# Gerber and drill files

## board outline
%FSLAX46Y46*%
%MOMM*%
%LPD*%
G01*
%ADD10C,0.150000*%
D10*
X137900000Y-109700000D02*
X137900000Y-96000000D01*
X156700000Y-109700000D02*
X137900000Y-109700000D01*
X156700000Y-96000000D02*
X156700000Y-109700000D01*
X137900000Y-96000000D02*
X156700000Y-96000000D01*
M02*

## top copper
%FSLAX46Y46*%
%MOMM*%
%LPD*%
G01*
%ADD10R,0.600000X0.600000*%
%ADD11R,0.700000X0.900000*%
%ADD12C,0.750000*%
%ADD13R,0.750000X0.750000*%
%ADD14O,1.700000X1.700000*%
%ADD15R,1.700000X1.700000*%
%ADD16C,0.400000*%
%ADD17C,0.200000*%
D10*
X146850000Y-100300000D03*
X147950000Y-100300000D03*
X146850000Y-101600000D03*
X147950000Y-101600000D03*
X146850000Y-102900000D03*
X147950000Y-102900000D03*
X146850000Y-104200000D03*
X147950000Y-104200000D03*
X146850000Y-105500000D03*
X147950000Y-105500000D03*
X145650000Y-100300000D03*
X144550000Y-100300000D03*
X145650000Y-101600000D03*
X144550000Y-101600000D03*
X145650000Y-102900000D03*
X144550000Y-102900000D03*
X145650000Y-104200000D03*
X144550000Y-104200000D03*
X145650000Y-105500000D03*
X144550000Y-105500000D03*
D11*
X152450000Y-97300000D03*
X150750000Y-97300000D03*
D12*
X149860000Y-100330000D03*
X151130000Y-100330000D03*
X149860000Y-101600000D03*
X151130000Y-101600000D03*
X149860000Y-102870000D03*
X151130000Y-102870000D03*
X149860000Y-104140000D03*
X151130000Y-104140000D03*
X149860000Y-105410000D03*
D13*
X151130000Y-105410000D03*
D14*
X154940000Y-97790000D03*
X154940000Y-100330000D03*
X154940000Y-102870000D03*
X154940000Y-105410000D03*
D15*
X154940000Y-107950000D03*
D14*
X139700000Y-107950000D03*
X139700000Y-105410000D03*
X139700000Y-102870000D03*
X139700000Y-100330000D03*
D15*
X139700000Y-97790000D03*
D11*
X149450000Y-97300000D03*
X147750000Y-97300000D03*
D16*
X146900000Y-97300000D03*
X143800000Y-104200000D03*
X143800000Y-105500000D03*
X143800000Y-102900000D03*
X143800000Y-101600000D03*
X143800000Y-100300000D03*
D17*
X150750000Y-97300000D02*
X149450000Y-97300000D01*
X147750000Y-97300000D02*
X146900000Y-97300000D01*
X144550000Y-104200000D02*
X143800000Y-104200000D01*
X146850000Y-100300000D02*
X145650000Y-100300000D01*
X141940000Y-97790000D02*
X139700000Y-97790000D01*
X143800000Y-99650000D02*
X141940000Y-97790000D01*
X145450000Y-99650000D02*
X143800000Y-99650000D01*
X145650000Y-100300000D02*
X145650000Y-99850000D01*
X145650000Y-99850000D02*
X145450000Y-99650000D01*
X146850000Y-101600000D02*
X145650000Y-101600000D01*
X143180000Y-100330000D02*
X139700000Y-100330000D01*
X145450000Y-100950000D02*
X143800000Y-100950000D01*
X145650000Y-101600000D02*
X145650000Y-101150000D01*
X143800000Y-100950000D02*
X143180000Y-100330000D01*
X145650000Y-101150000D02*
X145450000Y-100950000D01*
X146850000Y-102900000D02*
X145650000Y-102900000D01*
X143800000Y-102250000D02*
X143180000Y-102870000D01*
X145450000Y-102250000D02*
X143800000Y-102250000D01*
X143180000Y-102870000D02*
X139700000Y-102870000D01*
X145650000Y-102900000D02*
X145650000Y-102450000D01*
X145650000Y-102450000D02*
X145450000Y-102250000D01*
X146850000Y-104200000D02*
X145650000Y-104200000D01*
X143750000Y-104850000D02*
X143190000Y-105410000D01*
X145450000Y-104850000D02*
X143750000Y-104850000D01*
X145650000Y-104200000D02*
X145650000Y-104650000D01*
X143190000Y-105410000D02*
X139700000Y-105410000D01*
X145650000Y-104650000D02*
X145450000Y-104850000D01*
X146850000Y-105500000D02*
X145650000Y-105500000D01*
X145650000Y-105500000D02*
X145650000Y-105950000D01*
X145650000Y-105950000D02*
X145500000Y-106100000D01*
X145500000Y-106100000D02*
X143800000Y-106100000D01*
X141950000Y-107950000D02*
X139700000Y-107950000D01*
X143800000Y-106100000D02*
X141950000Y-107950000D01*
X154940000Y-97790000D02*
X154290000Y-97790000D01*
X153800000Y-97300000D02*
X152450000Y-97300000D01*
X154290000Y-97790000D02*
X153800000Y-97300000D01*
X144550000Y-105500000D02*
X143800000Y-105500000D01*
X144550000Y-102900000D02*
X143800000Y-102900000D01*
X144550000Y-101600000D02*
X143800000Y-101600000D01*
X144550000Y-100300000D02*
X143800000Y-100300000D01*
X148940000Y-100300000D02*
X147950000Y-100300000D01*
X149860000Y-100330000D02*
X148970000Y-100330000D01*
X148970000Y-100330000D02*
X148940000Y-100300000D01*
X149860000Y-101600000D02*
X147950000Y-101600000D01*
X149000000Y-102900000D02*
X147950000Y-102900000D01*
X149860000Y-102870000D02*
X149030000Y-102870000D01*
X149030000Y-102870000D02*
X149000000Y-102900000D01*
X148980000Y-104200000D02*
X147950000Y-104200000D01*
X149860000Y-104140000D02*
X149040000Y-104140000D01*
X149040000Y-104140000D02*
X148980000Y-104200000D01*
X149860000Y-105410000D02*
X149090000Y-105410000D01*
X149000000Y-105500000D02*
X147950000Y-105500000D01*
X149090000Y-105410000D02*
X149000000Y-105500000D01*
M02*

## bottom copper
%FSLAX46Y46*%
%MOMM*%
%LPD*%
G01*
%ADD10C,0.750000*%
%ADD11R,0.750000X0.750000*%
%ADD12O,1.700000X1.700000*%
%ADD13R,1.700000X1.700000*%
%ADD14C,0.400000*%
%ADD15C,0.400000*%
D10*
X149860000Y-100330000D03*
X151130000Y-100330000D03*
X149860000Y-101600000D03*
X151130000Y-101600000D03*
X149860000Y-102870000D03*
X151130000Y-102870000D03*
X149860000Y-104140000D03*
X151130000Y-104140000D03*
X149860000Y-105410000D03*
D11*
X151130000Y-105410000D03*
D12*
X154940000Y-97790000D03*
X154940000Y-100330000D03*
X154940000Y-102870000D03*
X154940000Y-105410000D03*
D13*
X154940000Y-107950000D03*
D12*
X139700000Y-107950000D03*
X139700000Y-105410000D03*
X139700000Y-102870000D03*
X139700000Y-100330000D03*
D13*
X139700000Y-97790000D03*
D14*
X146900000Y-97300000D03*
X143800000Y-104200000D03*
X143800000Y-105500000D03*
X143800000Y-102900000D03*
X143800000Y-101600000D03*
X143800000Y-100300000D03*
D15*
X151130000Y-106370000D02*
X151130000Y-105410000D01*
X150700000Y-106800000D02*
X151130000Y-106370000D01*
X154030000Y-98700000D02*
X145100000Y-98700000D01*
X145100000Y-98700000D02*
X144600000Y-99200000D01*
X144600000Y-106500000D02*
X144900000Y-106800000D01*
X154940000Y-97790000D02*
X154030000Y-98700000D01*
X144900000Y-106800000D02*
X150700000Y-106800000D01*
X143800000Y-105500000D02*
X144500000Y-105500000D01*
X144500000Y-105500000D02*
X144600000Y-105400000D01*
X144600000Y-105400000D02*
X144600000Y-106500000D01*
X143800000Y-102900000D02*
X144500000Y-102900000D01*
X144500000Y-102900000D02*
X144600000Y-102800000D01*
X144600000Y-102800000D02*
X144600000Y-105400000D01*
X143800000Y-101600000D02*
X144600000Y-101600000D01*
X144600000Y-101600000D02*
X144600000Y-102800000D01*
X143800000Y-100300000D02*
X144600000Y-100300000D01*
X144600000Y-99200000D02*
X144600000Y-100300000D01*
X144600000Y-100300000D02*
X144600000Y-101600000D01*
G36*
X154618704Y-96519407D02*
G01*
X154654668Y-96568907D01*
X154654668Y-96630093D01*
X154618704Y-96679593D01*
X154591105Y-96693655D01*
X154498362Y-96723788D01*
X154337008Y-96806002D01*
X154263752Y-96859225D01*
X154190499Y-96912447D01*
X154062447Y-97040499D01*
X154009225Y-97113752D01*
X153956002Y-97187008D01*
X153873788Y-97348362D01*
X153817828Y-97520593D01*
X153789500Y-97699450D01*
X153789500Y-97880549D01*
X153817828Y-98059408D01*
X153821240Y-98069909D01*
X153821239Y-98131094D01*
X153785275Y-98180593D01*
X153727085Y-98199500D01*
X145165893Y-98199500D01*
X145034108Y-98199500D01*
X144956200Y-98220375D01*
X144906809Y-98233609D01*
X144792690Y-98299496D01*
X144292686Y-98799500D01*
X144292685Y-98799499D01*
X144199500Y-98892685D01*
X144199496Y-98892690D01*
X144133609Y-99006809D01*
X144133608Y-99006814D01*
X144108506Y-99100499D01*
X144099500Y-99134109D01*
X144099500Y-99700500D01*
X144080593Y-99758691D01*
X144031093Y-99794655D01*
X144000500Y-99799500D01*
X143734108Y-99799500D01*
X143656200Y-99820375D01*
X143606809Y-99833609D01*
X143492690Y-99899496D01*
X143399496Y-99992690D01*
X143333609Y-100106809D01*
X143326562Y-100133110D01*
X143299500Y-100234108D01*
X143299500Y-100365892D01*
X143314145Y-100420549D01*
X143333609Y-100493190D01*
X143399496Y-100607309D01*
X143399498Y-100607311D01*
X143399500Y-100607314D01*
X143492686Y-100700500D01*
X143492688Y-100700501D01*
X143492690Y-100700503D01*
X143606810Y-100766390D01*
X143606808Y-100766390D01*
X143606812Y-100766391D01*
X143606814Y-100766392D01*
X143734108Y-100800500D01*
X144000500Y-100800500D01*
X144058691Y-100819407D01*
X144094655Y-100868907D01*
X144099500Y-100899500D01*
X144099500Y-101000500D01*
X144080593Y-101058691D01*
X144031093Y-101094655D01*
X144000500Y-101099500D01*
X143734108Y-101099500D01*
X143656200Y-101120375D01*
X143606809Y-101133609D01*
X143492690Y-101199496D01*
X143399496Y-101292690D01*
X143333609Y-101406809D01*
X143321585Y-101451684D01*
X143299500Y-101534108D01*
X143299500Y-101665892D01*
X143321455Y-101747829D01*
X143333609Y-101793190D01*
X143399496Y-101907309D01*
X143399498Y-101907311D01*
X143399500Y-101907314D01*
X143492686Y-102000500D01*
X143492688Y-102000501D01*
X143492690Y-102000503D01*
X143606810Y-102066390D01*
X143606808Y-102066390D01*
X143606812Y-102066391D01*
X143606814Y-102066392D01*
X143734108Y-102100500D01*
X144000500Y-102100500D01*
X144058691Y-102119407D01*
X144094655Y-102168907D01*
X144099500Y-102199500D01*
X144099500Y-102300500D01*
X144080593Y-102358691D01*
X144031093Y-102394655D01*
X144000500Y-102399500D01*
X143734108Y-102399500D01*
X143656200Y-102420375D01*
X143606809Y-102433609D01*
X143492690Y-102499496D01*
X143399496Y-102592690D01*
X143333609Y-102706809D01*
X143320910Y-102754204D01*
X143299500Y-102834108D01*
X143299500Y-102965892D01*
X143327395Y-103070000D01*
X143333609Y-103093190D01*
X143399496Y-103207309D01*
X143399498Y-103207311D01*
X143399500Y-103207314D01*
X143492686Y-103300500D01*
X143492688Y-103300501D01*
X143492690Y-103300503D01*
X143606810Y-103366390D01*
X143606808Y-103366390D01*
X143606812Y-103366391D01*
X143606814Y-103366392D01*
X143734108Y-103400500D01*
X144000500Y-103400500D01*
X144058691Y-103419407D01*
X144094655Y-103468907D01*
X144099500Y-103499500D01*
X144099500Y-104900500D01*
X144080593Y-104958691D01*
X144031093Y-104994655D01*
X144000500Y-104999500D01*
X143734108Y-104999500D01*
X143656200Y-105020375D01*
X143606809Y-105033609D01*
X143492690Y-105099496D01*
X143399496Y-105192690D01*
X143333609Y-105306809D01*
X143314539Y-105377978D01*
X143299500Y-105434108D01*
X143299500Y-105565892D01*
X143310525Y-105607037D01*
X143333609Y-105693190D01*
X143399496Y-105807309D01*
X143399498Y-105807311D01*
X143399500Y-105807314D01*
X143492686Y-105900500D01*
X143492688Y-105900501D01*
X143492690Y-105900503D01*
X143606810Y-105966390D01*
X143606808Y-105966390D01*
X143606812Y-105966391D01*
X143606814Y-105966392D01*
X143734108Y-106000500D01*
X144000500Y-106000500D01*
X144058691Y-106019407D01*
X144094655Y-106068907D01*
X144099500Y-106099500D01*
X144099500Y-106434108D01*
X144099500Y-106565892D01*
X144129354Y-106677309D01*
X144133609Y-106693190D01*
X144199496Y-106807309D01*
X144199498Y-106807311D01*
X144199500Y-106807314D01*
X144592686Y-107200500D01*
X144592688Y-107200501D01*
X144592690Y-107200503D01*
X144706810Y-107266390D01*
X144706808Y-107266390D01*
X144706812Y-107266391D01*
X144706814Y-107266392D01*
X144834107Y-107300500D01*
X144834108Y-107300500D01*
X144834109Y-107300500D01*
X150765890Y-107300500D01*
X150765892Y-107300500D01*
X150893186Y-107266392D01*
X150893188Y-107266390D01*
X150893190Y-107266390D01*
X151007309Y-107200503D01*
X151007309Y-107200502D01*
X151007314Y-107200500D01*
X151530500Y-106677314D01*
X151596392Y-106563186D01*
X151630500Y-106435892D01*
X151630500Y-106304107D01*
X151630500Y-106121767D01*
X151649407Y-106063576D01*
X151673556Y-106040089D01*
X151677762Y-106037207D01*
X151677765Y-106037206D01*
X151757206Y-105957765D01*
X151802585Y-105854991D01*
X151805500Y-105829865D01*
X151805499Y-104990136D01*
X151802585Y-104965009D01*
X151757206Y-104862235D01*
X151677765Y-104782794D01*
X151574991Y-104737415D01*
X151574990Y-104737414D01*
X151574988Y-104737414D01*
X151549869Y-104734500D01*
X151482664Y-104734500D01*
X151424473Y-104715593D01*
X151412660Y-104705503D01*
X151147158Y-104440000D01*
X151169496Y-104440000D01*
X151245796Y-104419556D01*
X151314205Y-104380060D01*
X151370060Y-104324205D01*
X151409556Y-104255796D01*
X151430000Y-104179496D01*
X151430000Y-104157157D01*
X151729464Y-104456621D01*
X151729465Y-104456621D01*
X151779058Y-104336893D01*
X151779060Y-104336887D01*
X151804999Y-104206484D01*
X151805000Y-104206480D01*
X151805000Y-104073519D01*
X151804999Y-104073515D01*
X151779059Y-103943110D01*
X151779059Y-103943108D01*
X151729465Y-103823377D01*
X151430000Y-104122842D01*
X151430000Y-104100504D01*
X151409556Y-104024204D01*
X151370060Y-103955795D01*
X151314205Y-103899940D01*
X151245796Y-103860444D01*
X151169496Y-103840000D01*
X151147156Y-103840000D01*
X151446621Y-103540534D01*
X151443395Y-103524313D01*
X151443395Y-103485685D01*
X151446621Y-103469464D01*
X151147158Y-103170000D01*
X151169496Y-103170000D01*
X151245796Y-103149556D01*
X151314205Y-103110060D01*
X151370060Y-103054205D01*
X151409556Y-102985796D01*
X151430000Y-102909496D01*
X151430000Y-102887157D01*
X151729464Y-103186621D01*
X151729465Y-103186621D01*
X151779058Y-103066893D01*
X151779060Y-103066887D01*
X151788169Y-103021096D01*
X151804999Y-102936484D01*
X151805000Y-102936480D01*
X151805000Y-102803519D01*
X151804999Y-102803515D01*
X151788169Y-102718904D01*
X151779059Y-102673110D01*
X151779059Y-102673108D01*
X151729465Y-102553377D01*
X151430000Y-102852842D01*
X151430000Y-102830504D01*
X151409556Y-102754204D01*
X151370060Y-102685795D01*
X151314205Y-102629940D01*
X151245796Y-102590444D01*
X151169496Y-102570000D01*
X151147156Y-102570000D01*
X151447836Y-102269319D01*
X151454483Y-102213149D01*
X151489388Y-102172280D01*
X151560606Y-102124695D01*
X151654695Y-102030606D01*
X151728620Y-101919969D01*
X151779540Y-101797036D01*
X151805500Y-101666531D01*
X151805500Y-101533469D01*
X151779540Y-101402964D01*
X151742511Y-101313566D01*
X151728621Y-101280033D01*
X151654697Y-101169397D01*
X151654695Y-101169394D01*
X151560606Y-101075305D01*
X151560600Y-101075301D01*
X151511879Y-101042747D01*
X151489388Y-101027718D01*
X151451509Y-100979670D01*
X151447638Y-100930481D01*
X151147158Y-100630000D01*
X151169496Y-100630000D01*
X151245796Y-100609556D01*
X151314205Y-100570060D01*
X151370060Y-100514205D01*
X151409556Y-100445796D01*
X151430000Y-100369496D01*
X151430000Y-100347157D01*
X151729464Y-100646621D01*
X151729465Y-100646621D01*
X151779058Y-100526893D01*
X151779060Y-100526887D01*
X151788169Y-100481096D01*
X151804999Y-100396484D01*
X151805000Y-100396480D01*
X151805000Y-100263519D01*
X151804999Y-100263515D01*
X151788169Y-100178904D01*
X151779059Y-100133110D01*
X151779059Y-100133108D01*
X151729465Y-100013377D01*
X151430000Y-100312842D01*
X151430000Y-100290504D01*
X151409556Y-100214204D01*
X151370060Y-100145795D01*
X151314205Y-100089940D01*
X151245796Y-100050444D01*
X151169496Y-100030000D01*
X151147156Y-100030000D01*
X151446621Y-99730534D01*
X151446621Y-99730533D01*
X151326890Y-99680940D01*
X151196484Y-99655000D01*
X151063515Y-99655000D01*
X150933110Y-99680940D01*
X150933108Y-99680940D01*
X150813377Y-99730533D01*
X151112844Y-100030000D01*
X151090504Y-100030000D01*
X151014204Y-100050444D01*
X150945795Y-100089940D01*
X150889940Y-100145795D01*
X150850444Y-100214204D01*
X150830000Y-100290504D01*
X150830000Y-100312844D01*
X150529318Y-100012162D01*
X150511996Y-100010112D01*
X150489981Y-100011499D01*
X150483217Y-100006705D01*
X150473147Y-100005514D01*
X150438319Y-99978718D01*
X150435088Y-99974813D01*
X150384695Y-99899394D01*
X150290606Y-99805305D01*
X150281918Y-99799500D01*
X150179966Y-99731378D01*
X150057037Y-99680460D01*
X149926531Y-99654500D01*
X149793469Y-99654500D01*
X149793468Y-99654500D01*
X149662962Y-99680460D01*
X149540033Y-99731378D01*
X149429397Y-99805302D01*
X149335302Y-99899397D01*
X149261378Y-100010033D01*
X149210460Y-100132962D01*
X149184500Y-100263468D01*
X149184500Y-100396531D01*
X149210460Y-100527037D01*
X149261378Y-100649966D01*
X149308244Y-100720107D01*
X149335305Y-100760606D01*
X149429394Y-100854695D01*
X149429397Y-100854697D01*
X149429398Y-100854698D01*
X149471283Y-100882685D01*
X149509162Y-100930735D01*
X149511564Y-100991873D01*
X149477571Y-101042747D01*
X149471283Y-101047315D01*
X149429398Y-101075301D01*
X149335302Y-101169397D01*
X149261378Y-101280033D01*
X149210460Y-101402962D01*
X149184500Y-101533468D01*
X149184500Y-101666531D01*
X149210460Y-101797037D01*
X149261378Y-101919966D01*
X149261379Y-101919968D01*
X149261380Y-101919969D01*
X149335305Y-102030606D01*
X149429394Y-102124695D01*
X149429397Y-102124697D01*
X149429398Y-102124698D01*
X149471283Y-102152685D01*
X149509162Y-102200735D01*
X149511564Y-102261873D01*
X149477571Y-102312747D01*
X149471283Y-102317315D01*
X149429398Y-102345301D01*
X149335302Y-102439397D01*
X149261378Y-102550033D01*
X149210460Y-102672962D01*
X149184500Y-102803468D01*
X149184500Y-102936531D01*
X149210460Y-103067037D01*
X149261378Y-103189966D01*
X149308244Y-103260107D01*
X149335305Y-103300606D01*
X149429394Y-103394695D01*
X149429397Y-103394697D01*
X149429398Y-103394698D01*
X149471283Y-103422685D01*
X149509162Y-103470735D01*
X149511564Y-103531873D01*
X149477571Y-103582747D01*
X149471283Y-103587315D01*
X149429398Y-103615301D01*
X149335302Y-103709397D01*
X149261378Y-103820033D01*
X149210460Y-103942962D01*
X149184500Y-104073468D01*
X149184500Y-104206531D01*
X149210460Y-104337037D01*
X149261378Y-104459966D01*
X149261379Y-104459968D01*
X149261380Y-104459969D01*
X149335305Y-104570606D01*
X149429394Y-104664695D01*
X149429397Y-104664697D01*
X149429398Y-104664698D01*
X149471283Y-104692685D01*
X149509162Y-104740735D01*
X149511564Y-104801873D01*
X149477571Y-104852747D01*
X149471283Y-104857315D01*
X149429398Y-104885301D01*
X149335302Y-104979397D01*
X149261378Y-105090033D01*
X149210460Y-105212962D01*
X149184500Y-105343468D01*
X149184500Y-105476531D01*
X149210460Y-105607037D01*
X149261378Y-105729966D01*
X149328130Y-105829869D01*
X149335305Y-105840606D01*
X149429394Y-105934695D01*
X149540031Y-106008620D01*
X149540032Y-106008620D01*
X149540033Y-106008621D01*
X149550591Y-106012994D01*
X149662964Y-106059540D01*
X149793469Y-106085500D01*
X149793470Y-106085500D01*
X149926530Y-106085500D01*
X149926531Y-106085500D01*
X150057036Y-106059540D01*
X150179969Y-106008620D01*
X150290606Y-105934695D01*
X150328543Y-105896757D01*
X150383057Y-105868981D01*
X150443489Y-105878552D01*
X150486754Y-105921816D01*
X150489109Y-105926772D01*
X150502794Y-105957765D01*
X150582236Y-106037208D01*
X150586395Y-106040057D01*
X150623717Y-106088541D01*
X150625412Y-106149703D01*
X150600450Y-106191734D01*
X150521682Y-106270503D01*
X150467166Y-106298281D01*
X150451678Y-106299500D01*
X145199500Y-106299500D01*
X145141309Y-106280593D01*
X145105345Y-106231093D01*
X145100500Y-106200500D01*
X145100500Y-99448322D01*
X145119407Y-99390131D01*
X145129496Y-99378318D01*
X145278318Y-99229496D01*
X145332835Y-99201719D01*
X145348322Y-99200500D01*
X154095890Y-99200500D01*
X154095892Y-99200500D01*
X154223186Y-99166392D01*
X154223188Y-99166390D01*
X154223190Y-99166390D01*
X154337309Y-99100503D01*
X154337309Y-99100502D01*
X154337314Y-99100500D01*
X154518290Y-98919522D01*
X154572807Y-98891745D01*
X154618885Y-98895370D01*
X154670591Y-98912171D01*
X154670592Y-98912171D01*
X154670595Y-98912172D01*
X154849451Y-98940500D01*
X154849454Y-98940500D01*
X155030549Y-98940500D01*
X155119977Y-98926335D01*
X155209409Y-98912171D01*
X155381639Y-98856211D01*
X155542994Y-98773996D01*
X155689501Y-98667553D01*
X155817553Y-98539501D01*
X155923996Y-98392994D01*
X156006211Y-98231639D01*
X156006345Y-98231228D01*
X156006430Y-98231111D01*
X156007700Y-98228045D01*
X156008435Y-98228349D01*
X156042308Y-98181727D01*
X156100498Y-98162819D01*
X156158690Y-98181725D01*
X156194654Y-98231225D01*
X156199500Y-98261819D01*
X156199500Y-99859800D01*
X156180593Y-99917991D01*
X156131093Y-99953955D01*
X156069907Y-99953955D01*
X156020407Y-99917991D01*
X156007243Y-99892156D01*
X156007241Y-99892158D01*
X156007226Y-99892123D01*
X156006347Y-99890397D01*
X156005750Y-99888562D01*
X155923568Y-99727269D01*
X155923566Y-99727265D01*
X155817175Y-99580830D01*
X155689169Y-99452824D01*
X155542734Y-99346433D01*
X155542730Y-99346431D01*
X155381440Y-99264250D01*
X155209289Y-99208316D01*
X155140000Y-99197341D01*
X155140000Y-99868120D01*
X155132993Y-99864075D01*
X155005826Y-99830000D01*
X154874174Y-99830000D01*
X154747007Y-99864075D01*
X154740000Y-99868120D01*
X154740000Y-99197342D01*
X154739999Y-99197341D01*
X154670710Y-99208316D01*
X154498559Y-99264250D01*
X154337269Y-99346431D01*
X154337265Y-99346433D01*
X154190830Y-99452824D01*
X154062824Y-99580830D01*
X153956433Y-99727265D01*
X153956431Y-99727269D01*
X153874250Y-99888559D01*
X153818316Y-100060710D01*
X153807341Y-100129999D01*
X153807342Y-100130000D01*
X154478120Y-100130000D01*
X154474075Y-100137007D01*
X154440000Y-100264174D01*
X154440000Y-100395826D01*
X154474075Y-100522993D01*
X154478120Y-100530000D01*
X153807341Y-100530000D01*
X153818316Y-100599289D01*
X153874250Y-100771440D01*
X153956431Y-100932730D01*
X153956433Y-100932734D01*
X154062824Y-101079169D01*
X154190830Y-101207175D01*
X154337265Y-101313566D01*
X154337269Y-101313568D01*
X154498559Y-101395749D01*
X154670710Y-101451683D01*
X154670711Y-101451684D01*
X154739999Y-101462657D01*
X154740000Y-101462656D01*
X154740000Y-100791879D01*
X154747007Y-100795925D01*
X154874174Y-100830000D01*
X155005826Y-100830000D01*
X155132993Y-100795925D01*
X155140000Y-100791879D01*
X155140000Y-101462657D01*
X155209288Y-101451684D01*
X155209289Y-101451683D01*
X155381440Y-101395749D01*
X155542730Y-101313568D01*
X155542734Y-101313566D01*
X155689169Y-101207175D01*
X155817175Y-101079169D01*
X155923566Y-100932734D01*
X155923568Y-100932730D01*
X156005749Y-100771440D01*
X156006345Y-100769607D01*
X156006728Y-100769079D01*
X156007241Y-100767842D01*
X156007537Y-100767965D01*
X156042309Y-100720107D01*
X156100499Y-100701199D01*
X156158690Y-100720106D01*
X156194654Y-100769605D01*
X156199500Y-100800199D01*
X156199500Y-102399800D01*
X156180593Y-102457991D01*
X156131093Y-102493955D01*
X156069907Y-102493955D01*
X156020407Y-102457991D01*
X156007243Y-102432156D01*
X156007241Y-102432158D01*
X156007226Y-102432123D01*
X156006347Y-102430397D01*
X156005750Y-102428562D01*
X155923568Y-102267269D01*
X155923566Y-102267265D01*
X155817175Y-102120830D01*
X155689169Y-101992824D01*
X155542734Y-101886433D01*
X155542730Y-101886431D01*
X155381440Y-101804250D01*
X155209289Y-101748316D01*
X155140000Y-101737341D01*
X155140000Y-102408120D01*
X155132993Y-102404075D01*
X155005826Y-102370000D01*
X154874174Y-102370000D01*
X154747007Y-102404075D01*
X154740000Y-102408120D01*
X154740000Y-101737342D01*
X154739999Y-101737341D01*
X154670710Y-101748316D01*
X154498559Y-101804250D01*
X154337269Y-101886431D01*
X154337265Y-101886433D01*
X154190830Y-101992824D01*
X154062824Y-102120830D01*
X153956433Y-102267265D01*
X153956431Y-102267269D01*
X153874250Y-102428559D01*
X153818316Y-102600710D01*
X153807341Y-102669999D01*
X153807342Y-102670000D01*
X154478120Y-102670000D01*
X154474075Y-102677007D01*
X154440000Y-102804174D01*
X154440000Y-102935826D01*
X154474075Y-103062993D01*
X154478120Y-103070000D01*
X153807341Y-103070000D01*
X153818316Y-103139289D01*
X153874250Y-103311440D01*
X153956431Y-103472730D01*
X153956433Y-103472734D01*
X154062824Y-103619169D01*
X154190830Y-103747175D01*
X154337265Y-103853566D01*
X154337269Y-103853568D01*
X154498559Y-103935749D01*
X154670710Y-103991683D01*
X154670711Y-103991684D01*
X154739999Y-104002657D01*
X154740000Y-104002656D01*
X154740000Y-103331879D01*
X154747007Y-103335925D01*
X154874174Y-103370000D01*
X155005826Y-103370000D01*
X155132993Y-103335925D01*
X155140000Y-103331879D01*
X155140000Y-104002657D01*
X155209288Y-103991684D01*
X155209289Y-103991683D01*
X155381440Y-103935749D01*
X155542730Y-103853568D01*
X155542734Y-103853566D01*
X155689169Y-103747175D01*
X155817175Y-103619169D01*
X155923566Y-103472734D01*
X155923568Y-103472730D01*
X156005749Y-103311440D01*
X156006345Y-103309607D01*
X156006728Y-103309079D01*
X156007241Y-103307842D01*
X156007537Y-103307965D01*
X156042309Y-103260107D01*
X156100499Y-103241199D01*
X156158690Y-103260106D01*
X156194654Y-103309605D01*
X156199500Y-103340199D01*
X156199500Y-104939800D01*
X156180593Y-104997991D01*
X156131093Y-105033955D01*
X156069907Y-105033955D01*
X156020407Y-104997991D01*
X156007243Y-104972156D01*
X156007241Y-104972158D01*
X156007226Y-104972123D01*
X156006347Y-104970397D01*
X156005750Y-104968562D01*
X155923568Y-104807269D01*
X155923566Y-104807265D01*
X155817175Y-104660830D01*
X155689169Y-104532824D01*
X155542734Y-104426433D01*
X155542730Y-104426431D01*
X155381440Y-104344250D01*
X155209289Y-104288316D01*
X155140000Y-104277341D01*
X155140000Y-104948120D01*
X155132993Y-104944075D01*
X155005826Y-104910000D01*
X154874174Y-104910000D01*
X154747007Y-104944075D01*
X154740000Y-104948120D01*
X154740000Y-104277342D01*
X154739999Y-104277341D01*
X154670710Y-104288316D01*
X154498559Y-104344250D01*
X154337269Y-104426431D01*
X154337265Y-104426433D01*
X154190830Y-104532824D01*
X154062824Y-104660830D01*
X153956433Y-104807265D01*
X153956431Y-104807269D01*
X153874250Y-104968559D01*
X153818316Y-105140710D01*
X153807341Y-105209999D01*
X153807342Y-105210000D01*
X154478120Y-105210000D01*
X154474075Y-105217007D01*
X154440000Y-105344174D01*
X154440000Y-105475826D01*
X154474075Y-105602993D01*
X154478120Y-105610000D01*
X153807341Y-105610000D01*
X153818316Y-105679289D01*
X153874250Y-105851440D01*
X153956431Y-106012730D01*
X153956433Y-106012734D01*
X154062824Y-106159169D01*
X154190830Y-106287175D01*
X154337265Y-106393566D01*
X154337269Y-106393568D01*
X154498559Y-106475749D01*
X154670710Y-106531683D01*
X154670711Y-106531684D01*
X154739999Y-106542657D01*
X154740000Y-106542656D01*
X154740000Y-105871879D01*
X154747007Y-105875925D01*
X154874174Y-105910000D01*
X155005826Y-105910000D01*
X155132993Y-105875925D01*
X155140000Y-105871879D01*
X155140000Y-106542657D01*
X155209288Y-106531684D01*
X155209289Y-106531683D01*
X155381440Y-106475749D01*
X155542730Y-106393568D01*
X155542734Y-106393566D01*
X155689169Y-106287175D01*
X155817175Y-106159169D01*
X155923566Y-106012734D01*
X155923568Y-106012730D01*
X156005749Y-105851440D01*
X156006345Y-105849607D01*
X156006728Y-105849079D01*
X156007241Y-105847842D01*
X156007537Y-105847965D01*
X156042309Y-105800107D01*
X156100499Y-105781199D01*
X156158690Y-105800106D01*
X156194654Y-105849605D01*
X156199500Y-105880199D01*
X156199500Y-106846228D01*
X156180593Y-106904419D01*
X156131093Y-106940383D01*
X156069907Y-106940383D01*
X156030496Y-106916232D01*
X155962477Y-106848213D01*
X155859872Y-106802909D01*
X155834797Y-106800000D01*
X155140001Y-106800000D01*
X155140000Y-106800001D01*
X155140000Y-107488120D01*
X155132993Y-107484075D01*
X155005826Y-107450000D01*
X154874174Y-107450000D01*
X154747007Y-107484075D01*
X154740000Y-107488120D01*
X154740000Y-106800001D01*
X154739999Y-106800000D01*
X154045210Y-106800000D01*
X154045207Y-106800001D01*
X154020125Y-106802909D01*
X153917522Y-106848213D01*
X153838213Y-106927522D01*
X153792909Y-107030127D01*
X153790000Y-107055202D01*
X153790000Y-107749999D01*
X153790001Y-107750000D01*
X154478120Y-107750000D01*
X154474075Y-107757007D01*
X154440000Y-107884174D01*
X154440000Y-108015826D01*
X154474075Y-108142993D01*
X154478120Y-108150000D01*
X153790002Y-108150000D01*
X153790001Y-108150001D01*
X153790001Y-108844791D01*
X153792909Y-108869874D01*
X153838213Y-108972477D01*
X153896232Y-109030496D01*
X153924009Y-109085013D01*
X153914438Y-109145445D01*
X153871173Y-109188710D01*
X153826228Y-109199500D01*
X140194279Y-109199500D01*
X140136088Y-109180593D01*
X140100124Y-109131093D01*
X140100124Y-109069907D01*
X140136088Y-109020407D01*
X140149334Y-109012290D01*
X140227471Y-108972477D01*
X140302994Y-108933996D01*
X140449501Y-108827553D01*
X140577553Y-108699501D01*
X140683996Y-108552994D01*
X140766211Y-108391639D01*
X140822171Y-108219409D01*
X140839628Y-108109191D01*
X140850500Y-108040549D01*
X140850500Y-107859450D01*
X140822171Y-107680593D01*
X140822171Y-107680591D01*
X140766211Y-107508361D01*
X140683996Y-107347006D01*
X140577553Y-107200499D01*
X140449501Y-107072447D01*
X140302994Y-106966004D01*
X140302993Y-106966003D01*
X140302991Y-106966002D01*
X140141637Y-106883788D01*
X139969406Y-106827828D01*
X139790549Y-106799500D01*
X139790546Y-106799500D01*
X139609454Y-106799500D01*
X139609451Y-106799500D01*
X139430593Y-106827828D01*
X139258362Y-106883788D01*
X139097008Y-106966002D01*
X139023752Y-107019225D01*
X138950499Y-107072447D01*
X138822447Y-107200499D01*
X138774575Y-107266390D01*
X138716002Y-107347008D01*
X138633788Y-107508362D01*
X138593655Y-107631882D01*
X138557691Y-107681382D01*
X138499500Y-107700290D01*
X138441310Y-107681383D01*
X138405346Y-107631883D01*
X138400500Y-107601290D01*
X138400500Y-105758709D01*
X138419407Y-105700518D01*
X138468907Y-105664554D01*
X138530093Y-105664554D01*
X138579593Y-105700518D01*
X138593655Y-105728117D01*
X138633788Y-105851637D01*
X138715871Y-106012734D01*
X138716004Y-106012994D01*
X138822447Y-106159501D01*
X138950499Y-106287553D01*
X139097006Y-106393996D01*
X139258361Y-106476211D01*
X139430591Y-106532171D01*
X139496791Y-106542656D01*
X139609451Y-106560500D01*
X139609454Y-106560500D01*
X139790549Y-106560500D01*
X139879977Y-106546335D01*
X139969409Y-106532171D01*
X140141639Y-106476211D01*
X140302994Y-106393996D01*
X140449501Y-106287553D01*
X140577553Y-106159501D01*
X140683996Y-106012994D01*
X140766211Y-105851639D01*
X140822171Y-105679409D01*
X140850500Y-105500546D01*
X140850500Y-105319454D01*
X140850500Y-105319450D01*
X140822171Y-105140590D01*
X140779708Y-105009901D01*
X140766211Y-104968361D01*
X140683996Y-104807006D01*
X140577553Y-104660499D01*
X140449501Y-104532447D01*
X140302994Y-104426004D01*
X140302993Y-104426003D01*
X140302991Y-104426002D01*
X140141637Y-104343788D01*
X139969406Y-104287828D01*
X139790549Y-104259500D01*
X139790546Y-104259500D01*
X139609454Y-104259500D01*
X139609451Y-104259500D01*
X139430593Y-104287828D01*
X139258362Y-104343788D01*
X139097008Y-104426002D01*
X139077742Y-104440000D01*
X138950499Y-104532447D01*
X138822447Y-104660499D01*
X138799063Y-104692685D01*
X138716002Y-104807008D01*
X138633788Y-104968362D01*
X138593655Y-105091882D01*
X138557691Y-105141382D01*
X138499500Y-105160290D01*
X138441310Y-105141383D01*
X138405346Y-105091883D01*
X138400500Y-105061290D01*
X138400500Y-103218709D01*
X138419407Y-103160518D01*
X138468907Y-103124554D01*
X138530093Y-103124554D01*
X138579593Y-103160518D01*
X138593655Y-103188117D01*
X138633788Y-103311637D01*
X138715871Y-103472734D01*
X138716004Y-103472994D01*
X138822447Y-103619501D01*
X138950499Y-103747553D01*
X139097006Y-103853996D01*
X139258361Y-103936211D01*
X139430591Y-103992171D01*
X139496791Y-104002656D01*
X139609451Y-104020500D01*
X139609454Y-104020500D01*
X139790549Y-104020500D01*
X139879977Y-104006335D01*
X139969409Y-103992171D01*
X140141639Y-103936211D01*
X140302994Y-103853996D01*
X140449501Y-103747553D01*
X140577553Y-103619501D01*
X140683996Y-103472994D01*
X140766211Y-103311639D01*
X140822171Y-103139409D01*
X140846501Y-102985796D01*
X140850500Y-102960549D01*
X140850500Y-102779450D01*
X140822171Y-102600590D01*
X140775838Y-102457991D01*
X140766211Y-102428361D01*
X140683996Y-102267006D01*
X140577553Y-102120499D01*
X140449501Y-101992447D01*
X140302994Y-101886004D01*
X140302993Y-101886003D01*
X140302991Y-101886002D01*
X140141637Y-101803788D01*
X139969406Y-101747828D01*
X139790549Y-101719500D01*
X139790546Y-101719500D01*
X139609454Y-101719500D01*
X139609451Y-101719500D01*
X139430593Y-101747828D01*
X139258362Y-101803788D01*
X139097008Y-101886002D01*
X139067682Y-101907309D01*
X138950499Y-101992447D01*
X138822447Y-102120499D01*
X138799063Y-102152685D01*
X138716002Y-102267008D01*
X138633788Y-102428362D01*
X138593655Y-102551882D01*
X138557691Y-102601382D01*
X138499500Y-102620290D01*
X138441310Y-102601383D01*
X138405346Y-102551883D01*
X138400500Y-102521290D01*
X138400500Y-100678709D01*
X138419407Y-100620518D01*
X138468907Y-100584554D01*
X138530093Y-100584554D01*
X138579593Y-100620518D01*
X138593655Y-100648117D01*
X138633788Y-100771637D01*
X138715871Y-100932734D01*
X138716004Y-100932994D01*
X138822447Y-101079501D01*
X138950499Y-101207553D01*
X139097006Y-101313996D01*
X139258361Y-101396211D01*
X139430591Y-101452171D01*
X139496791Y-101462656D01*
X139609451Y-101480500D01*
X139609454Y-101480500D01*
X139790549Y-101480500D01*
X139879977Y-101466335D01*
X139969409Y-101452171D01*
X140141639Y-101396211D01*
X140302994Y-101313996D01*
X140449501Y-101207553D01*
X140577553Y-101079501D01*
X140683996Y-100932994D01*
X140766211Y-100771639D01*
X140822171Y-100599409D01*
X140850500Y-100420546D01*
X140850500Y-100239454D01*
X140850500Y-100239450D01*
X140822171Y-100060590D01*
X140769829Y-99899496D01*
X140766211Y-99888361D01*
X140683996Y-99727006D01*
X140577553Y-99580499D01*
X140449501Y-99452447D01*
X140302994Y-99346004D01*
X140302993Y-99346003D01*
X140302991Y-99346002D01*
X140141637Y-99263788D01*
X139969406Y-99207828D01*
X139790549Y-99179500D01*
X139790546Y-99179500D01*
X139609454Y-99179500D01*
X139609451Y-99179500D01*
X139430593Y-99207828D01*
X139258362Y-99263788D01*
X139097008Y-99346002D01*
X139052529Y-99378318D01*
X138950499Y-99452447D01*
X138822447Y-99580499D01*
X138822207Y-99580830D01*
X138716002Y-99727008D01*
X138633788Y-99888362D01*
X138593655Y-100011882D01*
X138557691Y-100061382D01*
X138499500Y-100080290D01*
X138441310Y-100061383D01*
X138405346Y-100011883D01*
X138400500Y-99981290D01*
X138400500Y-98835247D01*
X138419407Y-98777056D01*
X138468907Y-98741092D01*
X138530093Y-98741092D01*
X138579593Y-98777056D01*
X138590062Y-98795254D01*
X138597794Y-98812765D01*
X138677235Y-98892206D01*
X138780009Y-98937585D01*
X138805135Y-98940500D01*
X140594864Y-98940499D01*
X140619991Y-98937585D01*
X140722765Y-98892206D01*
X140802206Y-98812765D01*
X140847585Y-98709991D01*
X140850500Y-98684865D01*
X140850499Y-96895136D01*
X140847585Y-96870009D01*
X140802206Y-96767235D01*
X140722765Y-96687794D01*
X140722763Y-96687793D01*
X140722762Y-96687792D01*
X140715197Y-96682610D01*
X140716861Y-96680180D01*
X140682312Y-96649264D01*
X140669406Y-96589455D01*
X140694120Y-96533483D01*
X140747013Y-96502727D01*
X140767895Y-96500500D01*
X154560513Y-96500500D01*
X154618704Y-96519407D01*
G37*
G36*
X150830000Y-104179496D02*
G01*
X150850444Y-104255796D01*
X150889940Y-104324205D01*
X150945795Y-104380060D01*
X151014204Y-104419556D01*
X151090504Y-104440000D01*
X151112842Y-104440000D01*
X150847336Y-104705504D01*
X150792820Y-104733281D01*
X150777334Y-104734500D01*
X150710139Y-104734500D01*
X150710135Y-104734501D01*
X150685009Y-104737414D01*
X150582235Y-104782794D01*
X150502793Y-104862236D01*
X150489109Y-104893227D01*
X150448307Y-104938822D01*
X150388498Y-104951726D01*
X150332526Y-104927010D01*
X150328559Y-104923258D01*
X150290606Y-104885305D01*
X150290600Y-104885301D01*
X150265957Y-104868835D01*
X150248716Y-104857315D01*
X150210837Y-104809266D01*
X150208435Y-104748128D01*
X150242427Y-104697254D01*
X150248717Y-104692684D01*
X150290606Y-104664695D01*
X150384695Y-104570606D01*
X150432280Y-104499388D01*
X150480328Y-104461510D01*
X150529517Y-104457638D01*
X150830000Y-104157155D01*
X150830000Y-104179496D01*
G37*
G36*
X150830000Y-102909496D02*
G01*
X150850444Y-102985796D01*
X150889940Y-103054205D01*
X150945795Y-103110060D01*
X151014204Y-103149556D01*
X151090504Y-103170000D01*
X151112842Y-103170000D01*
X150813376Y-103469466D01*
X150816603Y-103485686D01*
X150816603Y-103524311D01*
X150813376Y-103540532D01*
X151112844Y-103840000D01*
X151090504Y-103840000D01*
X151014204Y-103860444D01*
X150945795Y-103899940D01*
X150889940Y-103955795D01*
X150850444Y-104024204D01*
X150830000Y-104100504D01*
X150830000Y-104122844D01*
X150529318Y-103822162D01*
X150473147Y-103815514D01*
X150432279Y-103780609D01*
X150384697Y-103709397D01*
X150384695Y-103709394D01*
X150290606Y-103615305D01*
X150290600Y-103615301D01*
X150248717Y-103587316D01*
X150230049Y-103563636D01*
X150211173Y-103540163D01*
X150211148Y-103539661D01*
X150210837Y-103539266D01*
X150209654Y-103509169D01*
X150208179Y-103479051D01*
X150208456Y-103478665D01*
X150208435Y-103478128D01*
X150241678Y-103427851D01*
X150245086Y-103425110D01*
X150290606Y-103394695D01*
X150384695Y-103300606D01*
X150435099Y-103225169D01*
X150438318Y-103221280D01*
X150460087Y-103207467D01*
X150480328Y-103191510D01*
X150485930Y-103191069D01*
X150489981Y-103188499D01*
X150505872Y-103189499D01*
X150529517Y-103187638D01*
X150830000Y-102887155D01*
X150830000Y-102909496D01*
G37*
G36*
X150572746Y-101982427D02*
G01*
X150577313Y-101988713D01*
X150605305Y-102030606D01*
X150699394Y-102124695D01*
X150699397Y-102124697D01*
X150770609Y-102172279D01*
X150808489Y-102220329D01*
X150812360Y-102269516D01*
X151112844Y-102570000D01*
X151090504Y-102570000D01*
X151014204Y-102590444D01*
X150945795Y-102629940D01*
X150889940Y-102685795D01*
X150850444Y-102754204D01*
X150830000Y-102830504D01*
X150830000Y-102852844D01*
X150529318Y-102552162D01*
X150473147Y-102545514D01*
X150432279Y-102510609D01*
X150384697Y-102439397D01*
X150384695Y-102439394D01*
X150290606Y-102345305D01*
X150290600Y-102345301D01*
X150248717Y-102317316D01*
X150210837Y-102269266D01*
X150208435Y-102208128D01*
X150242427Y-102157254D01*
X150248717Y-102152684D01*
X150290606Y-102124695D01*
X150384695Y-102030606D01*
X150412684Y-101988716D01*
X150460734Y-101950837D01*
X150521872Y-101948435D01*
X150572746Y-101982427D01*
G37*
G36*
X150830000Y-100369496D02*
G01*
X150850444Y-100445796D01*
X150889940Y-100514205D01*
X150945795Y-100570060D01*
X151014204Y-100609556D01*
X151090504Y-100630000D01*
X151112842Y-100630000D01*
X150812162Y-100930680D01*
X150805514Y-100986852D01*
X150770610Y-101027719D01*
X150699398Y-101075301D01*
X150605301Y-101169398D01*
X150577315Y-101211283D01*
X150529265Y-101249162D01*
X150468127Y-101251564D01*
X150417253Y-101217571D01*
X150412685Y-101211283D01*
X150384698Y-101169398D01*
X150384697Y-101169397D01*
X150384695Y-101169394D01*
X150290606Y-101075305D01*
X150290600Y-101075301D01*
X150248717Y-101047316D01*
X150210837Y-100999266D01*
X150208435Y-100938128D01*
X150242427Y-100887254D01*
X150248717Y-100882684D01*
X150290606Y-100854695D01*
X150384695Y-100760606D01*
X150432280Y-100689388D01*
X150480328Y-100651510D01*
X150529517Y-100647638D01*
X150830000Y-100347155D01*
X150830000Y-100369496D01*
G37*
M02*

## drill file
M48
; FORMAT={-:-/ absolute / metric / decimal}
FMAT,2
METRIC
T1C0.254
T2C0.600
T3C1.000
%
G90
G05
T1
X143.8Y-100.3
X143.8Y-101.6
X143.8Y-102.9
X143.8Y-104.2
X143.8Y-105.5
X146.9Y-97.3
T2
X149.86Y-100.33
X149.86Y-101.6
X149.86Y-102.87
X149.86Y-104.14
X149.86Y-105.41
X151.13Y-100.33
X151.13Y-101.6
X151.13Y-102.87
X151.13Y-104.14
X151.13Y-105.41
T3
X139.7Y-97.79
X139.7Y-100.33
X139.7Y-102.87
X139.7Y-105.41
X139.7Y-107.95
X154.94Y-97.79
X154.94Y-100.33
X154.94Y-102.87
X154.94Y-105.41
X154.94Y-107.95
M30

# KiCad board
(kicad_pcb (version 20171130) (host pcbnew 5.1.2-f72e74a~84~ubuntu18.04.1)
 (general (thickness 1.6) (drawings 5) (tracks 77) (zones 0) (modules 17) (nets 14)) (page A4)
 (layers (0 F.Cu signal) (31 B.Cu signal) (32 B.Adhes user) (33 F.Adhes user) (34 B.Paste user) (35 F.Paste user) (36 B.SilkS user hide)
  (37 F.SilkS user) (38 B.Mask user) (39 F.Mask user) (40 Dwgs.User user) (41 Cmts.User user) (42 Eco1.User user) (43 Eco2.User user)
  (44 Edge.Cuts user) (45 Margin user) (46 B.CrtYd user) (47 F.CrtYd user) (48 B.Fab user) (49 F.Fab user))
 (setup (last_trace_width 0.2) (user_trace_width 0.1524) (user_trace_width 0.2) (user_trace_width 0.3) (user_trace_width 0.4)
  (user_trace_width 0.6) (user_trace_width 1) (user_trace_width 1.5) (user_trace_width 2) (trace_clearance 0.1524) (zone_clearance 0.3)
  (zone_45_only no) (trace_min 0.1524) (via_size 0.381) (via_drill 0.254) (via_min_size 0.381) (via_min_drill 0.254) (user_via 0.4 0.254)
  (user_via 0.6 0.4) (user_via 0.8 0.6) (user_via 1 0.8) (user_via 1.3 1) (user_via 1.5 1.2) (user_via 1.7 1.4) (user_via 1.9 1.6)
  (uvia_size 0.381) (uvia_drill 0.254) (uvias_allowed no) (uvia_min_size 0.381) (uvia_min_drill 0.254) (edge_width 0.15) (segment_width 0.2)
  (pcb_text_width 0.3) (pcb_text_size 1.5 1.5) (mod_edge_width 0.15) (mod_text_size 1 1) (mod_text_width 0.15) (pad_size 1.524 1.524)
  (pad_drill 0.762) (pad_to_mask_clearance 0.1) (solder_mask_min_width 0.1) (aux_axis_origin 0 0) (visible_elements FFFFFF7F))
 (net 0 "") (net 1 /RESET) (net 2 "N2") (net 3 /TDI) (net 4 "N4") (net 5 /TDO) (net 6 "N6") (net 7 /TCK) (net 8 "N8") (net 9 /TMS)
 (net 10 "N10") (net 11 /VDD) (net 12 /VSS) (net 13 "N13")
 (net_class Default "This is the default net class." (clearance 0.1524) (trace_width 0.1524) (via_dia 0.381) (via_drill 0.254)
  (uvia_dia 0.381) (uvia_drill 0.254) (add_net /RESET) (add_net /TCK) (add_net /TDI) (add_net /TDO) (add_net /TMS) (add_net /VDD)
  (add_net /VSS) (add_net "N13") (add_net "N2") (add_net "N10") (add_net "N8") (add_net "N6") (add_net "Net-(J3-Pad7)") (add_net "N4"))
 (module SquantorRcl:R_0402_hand (layer F.Cu) (at 147.4 100.3 180)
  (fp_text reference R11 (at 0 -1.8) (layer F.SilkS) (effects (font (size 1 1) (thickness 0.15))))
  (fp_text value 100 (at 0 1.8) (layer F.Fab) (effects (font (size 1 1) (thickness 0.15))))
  (pad 2 smd rect (at 0.55 0 180) (size 0.6 0.6) (layers F.Cu F.Paste F.Mask) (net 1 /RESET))
  (pad 1 smd rect (at -0.55 0 180) (size 0.6 0.6) (layers F.Cu F.Paste F.Mask) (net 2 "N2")))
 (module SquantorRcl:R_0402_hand (layer F.Cu) (at 147.4 101.6 180)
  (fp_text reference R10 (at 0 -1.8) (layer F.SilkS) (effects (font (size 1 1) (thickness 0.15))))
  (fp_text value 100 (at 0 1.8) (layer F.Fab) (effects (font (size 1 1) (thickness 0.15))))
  (pad 2 smd rect (at 0.55 0 180) (size 0.6 0.6) (layers F.Cu F.Paste F.Mask) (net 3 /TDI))
  (pad 1 smd rect (at -0.55 0 180) (size 0.6 0.6) (layers F.Cu F.Paste F.Mask) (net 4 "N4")))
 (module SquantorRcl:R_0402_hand (layer F.Cu) (at 147.4 102.9 180)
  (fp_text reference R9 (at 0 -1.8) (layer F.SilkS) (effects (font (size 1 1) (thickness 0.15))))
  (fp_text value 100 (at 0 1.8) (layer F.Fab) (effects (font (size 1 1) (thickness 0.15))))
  (pad 2 smd rect (at 0.55 0 180) (size 0.6 0.6) (layers F.Cu F.Paste F.Mask) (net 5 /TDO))
  (pad 1 smd rect (at -0.55 0 180) (size 0.6 0.6) (layers F.Cu F.Paste F.Mask) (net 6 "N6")))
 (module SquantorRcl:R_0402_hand (layer F.Cu) (at 147.4 104.2 180)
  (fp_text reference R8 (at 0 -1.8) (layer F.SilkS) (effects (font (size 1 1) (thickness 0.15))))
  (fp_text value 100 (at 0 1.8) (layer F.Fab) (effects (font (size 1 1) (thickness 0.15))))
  (pad 2 smd rect (at 0.55 0 180) (size 0.6 0.6) (layers F.Cu F.Paste F.Mask) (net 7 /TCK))
  (pad 1 smd rect (at -0.55 0 180) (size 0.6 0.6) (layers F.Cu F.Paste F.Mask) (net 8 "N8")))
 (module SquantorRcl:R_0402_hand (layer F.Cu) (at 147.4 105.5 180)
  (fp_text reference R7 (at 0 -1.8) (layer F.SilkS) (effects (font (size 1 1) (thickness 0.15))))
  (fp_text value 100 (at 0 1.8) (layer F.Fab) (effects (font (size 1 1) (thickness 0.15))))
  (pad 2 smd rect (at 0.55 0 180) (size 0.6 0.6) (layers F.Cu F.Paste F.Mask) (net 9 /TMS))
  (pad 1 smd rect (at -0.55 0 180) (size 0.6 0.6) (layers F.Cu F.Paste F.Mask) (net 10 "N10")))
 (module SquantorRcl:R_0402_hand (layer F.Cu) (at 145.1 100.3)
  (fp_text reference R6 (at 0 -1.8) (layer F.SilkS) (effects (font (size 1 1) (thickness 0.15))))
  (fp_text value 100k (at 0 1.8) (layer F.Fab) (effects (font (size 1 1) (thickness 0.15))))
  (pad 2 smd rect (at 0.55 0) (size 0.6 0.6) (layers F.Cu F.Paste F.Mask) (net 1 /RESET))
  (pad 1 smd rect (at -0.55 0) (size 0.6 0.6) (layers F.Cu F.Paste F.Mask) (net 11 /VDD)))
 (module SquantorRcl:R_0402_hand (layer F.Cu) (at 145.1 101.6)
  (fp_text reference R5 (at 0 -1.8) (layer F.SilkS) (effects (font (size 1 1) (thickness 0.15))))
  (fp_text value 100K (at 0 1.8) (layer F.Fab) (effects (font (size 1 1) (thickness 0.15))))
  (pad 2 smd rect (at 0.55 0) (size 0.6 0.6) (layers F.Cu F.Paste F.Mask) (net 3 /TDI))
  (pad 1 smd rect (at -0.55 0) (size 0.6 0.6) (layers F.Cu F.Paste F.Mask) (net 11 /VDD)))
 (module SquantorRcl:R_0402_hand (layer F.Cu) (at 145.1 102.9)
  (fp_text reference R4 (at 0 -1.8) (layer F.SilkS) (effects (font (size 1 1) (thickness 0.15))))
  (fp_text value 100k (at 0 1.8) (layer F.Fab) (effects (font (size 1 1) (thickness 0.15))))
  (pad 2 smd rect (at 0.55 0) (size 0.6 0.6) (layers F.Cu F.Paste F.Mask) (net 5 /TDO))
  (pad 1 smd rect (at -0.55 0) (size 0.6 0.6) (layers F.Cu F.Paste F.Mask) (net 11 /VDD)))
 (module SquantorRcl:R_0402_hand (layer F.Cu) (at 145.1 104.2)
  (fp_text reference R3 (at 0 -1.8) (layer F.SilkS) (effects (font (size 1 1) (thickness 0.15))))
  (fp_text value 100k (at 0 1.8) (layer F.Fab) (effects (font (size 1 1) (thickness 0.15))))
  (pad 2 smd rect (at 0.55 0) (size 0.6 0.6) (layers F.Cu F.Paste F.Mask) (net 7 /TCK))
  (pad 1 smd rect (at -0.55 0) (size 0.6 0.6) (layers F.Cu F.Paste F.Mask) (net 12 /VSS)))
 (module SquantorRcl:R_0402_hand (layer F.Cu) (at 145.1 105.5)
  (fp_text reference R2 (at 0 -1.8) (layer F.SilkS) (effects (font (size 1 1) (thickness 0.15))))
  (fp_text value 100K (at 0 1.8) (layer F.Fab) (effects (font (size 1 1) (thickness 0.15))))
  (pad 2 smd rect (at 0.55 0) (size 0.6 0.6) (layers F.Cu F.Paste F.Mask) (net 9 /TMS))
  (pad 1 smd rect (at -0.55 0) (size 0.6 0.6) (layers F.Cu F.Paste F.Mask) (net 11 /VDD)))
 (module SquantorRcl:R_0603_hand (layer F.Cu) (at 151.6 97.3)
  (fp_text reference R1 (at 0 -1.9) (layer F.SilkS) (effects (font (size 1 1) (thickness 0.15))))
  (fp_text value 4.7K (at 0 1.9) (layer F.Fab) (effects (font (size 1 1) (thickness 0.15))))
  (pad 2 smd rect (at 0.85 0) (size 0.7 0.9) (layers F.Cu F.Paste F.Mask) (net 11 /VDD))
  (pad 1 smd rect (at -0.85 0) (size 0.7 0.9) (layers F.Cu F.Paste F.Mask) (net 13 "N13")))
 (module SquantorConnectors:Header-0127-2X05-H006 (layer F.Cu) (at 150.495 102.87 90)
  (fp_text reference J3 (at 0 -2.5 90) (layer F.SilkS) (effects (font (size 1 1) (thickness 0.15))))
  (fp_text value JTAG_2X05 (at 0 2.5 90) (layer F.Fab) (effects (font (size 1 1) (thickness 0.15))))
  (pad 10 thru_hole circle (at 2.54 -0.635 90) (size 0.75 0.75) (drill 0.6) (layers *.Cu *.Mask) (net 2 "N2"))
  (pad 9 thru_hole circle (at 2.54 0.635 90) (size 0.75 0.75) (drill 0.6) (layers *.Cu *.Mask) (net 12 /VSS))
  (pad 8 thru_hole circle (at 1.27 -0.635 90) (size 0.75 0.75) (drill 0.6) (layers *.Cu *.Mask) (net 4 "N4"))
  (pad 7 thru_hole circle (at 1.27 0.635 90) (size 0.75 0.75) (drill 0.6) (layers *.Cu *.Mask))
  (pad 6 thru_hole circle (at 0 -0.635 90) (size 0.75 0.75) (drill 0.6) (layers *.Cu *.Mask) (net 6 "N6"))
  (pad 5 thru_hole circle (at 0 0.635 90) (size 0.75 0.75) (drill 0.6) (layers *.Cu *.Mask) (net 12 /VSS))
  (pad 4 thru_hole circle (at -1.27 -0.635 90) (size 0.75 0.75) (drill 0.6) (layers *.Cu *.Mask) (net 8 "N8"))
  (pad 3 thru_hole circle (at -1.27 0.635 90) (size 0.75 0.75) (drill 0.6) (layers *.Cu *.Mask) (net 12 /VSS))
  (pad 2 thru_hole circle (at -2.54 -0.635 90) (size 0.75 0.75) (drill 0.6) (layers *.Cu *.Mask) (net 10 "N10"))
  (pad 1 thru_hole rect (at -2.54 0.635 90) (size 0.75 0.75) (drill 0.6) (layers *.Cu *.Mask) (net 11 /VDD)))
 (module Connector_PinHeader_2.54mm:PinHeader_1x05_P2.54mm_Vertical (layer F.Cu) (at 154.94 107.95 180)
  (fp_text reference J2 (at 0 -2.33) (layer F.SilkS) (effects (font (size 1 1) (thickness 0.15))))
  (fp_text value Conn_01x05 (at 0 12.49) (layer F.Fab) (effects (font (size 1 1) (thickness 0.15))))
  (pad 5 thru_hole oval (at 0 10.16 180) (size 1.7 1.7) (drill 1) (layers *.Cu *.Mask) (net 11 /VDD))
  (pad 4 thru_hole oval (at 0 7.62 180) (size 1.7 1.7) (drill 1) (layers *.Cu *.Mask) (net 12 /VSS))
  (pad 3 thru_hole oval (at 0 5.08 180) (size 1.7 1.7) (drill 1) (layers *.Cu *.Mask) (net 12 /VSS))
  (pad 2 thru_hole oval (at 0 2.54 180) (size 1.7 1.7) (drill 1) (layers *.Cu *.Mask) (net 12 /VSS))
  (pad 1 thru_hole rect (at 0 0 180) (size 1.7 1.7) (drill 1) (layers *.Cu *.Mask) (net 12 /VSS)))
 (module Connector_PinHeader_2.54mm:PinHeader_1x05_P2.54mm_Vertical (layer F.Cu) (at 139.7 97.79)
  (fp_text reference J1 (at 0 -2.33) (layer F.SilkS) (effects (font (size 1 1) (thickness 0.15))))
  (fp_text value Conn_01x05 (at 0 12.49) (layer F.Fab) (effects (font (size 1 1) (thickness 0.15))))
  (pad 5 thru_hole oval (at 0 10.16) (size 1.7 1.7) (drill 1) (layers *.Cu *.Mask) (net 9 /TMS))
  (pad 4 thru_hole oval (at 0 7.62) (size 1.7 1.7) (drill 1) (layers *.Cu *.Mask) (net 7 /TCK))
  (pad 3 thru_hole oval (at 0 5.08) (size 1.7 1.7) (drill 1) (layers *.Cu *.Mask) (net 5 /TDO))
  (pad 2 thru_hole oval (at 0 2.54) (size 1.7 1.7) (drill 1) (layers *.Cu *.Mask) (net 3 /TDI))
  (pad 1 thru_hole rect (at 0 0) (size 1.7 1.7) (drill 1) (layers *.Cu *.Mask) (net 1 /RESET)))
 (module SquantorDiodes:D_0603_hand (layer F.Cu) (at 148.6 97.3)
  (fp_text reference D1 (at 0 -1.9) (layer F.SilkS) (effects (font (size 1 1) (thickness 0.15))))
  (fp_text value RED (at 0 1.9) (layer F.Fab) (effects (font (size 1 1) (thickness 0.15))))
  (pad 2 smd rect (at 0.85 0) (size 0.7 0.9) (layers F.Cu F.Paste F.Mask) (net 13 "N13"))
  (pad 1 smd rect (at -0.85 0) (size 0.7 0.9) (layers F.Cu F.Paste F.Mask) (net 12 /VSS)))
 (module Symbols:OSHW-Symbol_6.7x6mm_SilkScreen (layer B.Cu) (at 148 101)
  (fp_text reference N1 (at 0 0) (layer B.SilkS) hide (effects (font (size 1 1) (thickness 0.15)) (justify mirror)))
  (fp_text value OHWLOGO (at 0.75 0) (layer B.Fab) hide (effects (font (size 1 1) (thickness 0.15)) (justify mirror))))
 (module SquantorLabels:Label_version (layer B.Cu) (at 148.9 104.8)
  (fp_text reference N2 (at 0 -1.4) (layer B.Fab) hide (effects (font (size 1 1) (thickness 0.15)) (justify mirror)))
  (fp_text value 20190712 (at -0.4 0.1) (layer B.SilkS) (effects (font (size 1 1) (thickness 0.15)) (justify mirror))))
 (gr_line (start 137.9 109.7) (end 137.9 96) (layer Edge.Cuts) (width 0.15))
 (gr_line (start 156.7 109.7) (end 137.9 109.7) (layer Edge.Cuts) (width 0.15))
 (gr_line (start 156.7 96) (end 156.7 109.7) (layer Edge.Cuts) (width 0.15))
 (gr_line (start 137.9 96) (end 156.7 96) (layer Edge.Cuts) (width 0.15))
 (segment (start 150.75 97.3) (end 149.45 97.3) (width 0.2) (layer F.Cu) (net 13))
 (via (at 146.9 97.3) (size 0.4) (drill 0.254) (layers F.Cu B.Cu) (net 12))
 (segment (start 147.75 97.3) (end 146.9 97.3) (width 0.2) (layer F.Cu) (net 12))
 (via (at 143.8 104.2) (size 0.4) (drill 0.254) (layers F.Cu B.Cu) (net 12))
 (segment (start 144.55 104.2) (end 143.8 104.2) (width 0.2) (layer F.Cu) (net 12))
 (segment (start 146.85 100.3) (end 145.65 100.3) (width 0.2) (layer F.Cu) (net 1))
 (segment (start 141.94 97.79) (end 139.7 97.79) (width 0.2) (layer F.Cu) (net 1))
 (segment (start 143.8 99.65) (end 141.94 97.79) (width 0.2) (layer F.Cu) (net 1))
 (segment (start 145.45 99.65) (end 143.8 99.65) (width 0.2) (layer F.Cu) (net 1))
 (segment (start 145.65 100.3) (end 145.65 99.85) (width 0.2) (layer F.Cu) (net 1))
 (segment (start 145.65 99.85) (end 145.45 99.65) (width 0.2) (layer F.Cu) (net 1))
 (segment (start 146.85 101.6) (end 145.65 101.6) (width 0.2) (layer F.Cu) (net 3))
 (segment (start 143.18 100.33) (end 139.7 100.33) (width 0.2) (layer F.Cu) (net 3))
 (segment (start 145.45 100.95) (end 143.8 100.95) (width 0.2) (layer F.Cu) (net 3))
 (segment (start 145.65 101.6) (end 145.65 101.15) (width 0.2) (layer F.Cu) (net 3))
 (segment (start 143.8 100.95) (end 143.18 100.33) (width 0.2) (layer F.Cu) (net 3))
 (segment (start 145.65 101.15) (end 145.45 100.95) (width 0.2) (layer F.Cu) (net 3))
 (segment (start 146.85 102.9) (end 145.65 102.9) (width 0.2) (layer F.Cu) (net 5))
 (segment (start 143.8 102.25) (end 143.18 102.87) (width 0.2) (layer F.Cu) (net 5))
 (segment (start 145.45 102.25) (end 143.8 102.25) (width 0.2) (layer F.Cu) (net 5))
 (segment (start 143.18 102.87) (end 139.7 102.87) (width 0.2) (layer F.Cu) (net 5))
 (segment (start 145.65 102.9) (end 145.65 102.45) (width 0.2) (layer F.Cu) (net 5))
 (segment (start 145.65 102.45) (end 145.45 102.25) (width 0.2) (layer F.Cu) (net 5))
 (segment (start 146.85 104.2) (end 145.65 104.2) (width 0.2) (layer F.Cu) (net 7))
 (segment (start 143.75 104.85) (end 143.19 105.41) (width 0.2) (layer F.Cu) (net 7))
 (segment (start 145.45 104.85) (end 143.75 104.85) (width 0.2) (layer F.Cu) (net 7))
 (segment (start 145.65 104.2) (end 145.65 104.65) (width 0.2) (layer F.Cu) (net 7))
 (segment (start 143.19 105.41) (end 139.7 105.41) (width 0.2) (layer F.Cu) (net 7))
 (segment (start 145.65 104.65) (end 145.45 104.85) (width 0.2) (layer F.Cu) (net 7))
 (segment (start 146.85 105.5) (end 145.65 105.5) (width 0.2) (layer F.Cu) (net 9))
 (segment (start 145.65 105.5) (end 145.65 105.95) (width 0.2) (layer F.Cu) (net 9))
 (segment (start 145.65 105.95) (end 145.5 106.1) (width 0.2) (layer F.Cu) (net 9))
 (segment (start 145.5 106.1) (end 143.8 106.1) (width 0.2) (layer F.Cu) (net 9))
 (segment (start 141.95 107.95) (end 139.7 107.95) (width 0.2) (layer F.Cu) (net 9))
 (segment (start 143.8 106.1) (end 141.95 107.95) (width 0.2) (layer F.Cu) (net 9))
 (segment (start 154.94 97.79) (end 154.29 97.79) (width 0.2) (layer F.Cu) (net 11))
 (segment (start 153.8 97.3) (end 152.45 97.3) (width 0.2) (layer F.Cu) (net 11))
 (segment (start 154.29 97.79) (end 153.8 97.3) (width 0.2) (layer F.Cu) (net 11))
 (via (at 143.8 105.5) (size 0.4) (drill 0.254) (layers F.Cu B.Cu) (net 11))
 (segment (start 144.55 105.5) (end 143.8 105.5) (width 0.2) (layer F.Cu) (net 11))
 (via (at 143.8 102.9) (size 0.4) (drill 0.254) (layers F.Cu B.Cu) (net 11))
 (segment (start 144.55 102.9) (end 143.8 102.9) (width 0.2) (layer F.Cu) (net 11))
 (via (at 143.8 101.6) (size 0.4) (drill 0.254) (layers F.Cu B.Cu) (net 11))
 (segment (start 144.55 101.6) (end 143.8 101.6) (width 0.2) (layer F.Cu) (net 11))
 (via (at 143.8 100.3) (size 0.4) (drill 0.254) (layers F.Cu B.Cu) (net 11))
 (segment (start 144.55 100.3) (end 143.8 100.3) (width 0.2) (layer F.Cu) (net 11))
 (segment (start 151.13 106.37) (end 151.13 105.41) (width 0.4) (layer B.Cu) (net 11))
 (segment (start 150.7 106.8) (end 151.13 106.37) (width 0.4) (layer B.Cu) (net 11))
 (segment (start 154.03 98.7) (end 145.1 98.7) (width 0.4) (layer B.Cu) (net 11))
 (segment (start 145.1 98.7) (end 144.6 99.2) (width 0.4) (layer B.Cu) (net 11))
 (segment (start 144.6 106.5) (end 144.9 106.8) (width 0.4) (layer B.Cu) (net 11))
 (segment (start 154.94 97.79) (end 154.03 98.7) (width 0.4) (layer B.Cu) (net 11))
 (segment (start 144.9 106.8) (end 150.7 106.8) (width 0.4) (layer B.Cu) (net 11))
 (segment (start 143.8 105.5) (end 144.5 105.5) (width 0.4) (layer B.Cu) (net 11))
 (segment (start 144.5 105.5) (end 144.6 105.4) (width 0.4) (layer B.Cu) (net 11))
 (segment (start 144.6 105.4) (end 144.6 106.5) (width 0.4) (layer B.Cu) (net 11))
 (segment (start 143.8 102.9) (end 144.5 102.9) (width 0.4) (layer B.Cu) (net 11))
 (segment (start 144.5 102.9) (end 144.6 102.8) (width 0.4) (layer B.Cu) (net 11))
 (segment (start 144.6 102.8) (end 144.6 105.4) (width 0.4) (layer B.Cu) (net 11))
 (segment (start 143.8 101.6) (end 144.6 101.6) (width 0.4) (layer B.Cu) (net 11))
 (segment (start 144.6 101.6) (end 144.6 102.8) (width 0.4) (layer B.Cu) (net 11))
 (segment (start 143.8 100.3) (end 144.6 100.3) (width 0.4) (layer B.Cu) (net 11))
 (segment (start 144.6 99.2) (end 144.6 100.3) (width 0.4) (layer B.Cu) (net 11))
 (segment (start 144.6 100.3) (end 144.6 101.6) (width 0.4) (layer B.Cu) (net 11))
 (segment (start 148.94 100.3) (end 147.95 100.3) (width 0.2) (layer F.Cu) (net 2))
 (segment (start 149.86 100.33) (end 148.97 100.33) (width 0.2) (layer F.Cu) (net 2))
 (segment (start 148.97 100.33) (end 148.94 100.3) (width 0.2) (layer F.Cu) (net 2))
 (segment (start 149.86 101.6) (end 147.95 101.6) (width 0.2) (layer F.Cu) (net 4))
 (segment (start 149 102.9) (end 147.95 102.9) (width 0.2) (layer F.Cu) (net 6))
 (segment (start 149.86 102.87) (end 149.03 102.87) (width 0.2) (layer F.Cu) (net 6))
 (segment (start 149.03 102.87) (end 149 102.9) (width 0.2) (layer F.Cu) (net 6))
 (segment (start 148.98 104.2) (end 147.95 104.2) (width 0.2) (layer F.Cu) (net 8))
 (segment (start 149.86 104.14) (end 149.04 104.14) (width 0.2) (layer F.Cu) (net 8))
 (segment (start 149.04 104.14) (end 148.98 104.2) (width 0.2) (layer F.Cu) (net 8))
 (segment (start 149.86 105.41) (end 149.09 105.41) (width 0.2) (layer F.Cu) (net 10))
 (segment (start 149 105.5) (end 147.95 105.5) (width 0.2) (layer F.Cu) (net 10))
 (segment (start 149.09 105.41) (end 149 105.5) (width 0.2) (layer F.Cu) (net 10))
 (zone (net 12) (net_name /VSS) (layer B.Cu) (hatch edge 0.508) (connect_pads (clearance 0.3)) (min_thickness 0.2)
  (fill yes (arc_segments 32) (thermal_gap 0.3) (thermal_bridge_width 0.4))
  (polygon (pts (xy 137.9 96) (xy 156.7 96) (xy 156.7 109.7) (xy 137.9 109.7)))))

